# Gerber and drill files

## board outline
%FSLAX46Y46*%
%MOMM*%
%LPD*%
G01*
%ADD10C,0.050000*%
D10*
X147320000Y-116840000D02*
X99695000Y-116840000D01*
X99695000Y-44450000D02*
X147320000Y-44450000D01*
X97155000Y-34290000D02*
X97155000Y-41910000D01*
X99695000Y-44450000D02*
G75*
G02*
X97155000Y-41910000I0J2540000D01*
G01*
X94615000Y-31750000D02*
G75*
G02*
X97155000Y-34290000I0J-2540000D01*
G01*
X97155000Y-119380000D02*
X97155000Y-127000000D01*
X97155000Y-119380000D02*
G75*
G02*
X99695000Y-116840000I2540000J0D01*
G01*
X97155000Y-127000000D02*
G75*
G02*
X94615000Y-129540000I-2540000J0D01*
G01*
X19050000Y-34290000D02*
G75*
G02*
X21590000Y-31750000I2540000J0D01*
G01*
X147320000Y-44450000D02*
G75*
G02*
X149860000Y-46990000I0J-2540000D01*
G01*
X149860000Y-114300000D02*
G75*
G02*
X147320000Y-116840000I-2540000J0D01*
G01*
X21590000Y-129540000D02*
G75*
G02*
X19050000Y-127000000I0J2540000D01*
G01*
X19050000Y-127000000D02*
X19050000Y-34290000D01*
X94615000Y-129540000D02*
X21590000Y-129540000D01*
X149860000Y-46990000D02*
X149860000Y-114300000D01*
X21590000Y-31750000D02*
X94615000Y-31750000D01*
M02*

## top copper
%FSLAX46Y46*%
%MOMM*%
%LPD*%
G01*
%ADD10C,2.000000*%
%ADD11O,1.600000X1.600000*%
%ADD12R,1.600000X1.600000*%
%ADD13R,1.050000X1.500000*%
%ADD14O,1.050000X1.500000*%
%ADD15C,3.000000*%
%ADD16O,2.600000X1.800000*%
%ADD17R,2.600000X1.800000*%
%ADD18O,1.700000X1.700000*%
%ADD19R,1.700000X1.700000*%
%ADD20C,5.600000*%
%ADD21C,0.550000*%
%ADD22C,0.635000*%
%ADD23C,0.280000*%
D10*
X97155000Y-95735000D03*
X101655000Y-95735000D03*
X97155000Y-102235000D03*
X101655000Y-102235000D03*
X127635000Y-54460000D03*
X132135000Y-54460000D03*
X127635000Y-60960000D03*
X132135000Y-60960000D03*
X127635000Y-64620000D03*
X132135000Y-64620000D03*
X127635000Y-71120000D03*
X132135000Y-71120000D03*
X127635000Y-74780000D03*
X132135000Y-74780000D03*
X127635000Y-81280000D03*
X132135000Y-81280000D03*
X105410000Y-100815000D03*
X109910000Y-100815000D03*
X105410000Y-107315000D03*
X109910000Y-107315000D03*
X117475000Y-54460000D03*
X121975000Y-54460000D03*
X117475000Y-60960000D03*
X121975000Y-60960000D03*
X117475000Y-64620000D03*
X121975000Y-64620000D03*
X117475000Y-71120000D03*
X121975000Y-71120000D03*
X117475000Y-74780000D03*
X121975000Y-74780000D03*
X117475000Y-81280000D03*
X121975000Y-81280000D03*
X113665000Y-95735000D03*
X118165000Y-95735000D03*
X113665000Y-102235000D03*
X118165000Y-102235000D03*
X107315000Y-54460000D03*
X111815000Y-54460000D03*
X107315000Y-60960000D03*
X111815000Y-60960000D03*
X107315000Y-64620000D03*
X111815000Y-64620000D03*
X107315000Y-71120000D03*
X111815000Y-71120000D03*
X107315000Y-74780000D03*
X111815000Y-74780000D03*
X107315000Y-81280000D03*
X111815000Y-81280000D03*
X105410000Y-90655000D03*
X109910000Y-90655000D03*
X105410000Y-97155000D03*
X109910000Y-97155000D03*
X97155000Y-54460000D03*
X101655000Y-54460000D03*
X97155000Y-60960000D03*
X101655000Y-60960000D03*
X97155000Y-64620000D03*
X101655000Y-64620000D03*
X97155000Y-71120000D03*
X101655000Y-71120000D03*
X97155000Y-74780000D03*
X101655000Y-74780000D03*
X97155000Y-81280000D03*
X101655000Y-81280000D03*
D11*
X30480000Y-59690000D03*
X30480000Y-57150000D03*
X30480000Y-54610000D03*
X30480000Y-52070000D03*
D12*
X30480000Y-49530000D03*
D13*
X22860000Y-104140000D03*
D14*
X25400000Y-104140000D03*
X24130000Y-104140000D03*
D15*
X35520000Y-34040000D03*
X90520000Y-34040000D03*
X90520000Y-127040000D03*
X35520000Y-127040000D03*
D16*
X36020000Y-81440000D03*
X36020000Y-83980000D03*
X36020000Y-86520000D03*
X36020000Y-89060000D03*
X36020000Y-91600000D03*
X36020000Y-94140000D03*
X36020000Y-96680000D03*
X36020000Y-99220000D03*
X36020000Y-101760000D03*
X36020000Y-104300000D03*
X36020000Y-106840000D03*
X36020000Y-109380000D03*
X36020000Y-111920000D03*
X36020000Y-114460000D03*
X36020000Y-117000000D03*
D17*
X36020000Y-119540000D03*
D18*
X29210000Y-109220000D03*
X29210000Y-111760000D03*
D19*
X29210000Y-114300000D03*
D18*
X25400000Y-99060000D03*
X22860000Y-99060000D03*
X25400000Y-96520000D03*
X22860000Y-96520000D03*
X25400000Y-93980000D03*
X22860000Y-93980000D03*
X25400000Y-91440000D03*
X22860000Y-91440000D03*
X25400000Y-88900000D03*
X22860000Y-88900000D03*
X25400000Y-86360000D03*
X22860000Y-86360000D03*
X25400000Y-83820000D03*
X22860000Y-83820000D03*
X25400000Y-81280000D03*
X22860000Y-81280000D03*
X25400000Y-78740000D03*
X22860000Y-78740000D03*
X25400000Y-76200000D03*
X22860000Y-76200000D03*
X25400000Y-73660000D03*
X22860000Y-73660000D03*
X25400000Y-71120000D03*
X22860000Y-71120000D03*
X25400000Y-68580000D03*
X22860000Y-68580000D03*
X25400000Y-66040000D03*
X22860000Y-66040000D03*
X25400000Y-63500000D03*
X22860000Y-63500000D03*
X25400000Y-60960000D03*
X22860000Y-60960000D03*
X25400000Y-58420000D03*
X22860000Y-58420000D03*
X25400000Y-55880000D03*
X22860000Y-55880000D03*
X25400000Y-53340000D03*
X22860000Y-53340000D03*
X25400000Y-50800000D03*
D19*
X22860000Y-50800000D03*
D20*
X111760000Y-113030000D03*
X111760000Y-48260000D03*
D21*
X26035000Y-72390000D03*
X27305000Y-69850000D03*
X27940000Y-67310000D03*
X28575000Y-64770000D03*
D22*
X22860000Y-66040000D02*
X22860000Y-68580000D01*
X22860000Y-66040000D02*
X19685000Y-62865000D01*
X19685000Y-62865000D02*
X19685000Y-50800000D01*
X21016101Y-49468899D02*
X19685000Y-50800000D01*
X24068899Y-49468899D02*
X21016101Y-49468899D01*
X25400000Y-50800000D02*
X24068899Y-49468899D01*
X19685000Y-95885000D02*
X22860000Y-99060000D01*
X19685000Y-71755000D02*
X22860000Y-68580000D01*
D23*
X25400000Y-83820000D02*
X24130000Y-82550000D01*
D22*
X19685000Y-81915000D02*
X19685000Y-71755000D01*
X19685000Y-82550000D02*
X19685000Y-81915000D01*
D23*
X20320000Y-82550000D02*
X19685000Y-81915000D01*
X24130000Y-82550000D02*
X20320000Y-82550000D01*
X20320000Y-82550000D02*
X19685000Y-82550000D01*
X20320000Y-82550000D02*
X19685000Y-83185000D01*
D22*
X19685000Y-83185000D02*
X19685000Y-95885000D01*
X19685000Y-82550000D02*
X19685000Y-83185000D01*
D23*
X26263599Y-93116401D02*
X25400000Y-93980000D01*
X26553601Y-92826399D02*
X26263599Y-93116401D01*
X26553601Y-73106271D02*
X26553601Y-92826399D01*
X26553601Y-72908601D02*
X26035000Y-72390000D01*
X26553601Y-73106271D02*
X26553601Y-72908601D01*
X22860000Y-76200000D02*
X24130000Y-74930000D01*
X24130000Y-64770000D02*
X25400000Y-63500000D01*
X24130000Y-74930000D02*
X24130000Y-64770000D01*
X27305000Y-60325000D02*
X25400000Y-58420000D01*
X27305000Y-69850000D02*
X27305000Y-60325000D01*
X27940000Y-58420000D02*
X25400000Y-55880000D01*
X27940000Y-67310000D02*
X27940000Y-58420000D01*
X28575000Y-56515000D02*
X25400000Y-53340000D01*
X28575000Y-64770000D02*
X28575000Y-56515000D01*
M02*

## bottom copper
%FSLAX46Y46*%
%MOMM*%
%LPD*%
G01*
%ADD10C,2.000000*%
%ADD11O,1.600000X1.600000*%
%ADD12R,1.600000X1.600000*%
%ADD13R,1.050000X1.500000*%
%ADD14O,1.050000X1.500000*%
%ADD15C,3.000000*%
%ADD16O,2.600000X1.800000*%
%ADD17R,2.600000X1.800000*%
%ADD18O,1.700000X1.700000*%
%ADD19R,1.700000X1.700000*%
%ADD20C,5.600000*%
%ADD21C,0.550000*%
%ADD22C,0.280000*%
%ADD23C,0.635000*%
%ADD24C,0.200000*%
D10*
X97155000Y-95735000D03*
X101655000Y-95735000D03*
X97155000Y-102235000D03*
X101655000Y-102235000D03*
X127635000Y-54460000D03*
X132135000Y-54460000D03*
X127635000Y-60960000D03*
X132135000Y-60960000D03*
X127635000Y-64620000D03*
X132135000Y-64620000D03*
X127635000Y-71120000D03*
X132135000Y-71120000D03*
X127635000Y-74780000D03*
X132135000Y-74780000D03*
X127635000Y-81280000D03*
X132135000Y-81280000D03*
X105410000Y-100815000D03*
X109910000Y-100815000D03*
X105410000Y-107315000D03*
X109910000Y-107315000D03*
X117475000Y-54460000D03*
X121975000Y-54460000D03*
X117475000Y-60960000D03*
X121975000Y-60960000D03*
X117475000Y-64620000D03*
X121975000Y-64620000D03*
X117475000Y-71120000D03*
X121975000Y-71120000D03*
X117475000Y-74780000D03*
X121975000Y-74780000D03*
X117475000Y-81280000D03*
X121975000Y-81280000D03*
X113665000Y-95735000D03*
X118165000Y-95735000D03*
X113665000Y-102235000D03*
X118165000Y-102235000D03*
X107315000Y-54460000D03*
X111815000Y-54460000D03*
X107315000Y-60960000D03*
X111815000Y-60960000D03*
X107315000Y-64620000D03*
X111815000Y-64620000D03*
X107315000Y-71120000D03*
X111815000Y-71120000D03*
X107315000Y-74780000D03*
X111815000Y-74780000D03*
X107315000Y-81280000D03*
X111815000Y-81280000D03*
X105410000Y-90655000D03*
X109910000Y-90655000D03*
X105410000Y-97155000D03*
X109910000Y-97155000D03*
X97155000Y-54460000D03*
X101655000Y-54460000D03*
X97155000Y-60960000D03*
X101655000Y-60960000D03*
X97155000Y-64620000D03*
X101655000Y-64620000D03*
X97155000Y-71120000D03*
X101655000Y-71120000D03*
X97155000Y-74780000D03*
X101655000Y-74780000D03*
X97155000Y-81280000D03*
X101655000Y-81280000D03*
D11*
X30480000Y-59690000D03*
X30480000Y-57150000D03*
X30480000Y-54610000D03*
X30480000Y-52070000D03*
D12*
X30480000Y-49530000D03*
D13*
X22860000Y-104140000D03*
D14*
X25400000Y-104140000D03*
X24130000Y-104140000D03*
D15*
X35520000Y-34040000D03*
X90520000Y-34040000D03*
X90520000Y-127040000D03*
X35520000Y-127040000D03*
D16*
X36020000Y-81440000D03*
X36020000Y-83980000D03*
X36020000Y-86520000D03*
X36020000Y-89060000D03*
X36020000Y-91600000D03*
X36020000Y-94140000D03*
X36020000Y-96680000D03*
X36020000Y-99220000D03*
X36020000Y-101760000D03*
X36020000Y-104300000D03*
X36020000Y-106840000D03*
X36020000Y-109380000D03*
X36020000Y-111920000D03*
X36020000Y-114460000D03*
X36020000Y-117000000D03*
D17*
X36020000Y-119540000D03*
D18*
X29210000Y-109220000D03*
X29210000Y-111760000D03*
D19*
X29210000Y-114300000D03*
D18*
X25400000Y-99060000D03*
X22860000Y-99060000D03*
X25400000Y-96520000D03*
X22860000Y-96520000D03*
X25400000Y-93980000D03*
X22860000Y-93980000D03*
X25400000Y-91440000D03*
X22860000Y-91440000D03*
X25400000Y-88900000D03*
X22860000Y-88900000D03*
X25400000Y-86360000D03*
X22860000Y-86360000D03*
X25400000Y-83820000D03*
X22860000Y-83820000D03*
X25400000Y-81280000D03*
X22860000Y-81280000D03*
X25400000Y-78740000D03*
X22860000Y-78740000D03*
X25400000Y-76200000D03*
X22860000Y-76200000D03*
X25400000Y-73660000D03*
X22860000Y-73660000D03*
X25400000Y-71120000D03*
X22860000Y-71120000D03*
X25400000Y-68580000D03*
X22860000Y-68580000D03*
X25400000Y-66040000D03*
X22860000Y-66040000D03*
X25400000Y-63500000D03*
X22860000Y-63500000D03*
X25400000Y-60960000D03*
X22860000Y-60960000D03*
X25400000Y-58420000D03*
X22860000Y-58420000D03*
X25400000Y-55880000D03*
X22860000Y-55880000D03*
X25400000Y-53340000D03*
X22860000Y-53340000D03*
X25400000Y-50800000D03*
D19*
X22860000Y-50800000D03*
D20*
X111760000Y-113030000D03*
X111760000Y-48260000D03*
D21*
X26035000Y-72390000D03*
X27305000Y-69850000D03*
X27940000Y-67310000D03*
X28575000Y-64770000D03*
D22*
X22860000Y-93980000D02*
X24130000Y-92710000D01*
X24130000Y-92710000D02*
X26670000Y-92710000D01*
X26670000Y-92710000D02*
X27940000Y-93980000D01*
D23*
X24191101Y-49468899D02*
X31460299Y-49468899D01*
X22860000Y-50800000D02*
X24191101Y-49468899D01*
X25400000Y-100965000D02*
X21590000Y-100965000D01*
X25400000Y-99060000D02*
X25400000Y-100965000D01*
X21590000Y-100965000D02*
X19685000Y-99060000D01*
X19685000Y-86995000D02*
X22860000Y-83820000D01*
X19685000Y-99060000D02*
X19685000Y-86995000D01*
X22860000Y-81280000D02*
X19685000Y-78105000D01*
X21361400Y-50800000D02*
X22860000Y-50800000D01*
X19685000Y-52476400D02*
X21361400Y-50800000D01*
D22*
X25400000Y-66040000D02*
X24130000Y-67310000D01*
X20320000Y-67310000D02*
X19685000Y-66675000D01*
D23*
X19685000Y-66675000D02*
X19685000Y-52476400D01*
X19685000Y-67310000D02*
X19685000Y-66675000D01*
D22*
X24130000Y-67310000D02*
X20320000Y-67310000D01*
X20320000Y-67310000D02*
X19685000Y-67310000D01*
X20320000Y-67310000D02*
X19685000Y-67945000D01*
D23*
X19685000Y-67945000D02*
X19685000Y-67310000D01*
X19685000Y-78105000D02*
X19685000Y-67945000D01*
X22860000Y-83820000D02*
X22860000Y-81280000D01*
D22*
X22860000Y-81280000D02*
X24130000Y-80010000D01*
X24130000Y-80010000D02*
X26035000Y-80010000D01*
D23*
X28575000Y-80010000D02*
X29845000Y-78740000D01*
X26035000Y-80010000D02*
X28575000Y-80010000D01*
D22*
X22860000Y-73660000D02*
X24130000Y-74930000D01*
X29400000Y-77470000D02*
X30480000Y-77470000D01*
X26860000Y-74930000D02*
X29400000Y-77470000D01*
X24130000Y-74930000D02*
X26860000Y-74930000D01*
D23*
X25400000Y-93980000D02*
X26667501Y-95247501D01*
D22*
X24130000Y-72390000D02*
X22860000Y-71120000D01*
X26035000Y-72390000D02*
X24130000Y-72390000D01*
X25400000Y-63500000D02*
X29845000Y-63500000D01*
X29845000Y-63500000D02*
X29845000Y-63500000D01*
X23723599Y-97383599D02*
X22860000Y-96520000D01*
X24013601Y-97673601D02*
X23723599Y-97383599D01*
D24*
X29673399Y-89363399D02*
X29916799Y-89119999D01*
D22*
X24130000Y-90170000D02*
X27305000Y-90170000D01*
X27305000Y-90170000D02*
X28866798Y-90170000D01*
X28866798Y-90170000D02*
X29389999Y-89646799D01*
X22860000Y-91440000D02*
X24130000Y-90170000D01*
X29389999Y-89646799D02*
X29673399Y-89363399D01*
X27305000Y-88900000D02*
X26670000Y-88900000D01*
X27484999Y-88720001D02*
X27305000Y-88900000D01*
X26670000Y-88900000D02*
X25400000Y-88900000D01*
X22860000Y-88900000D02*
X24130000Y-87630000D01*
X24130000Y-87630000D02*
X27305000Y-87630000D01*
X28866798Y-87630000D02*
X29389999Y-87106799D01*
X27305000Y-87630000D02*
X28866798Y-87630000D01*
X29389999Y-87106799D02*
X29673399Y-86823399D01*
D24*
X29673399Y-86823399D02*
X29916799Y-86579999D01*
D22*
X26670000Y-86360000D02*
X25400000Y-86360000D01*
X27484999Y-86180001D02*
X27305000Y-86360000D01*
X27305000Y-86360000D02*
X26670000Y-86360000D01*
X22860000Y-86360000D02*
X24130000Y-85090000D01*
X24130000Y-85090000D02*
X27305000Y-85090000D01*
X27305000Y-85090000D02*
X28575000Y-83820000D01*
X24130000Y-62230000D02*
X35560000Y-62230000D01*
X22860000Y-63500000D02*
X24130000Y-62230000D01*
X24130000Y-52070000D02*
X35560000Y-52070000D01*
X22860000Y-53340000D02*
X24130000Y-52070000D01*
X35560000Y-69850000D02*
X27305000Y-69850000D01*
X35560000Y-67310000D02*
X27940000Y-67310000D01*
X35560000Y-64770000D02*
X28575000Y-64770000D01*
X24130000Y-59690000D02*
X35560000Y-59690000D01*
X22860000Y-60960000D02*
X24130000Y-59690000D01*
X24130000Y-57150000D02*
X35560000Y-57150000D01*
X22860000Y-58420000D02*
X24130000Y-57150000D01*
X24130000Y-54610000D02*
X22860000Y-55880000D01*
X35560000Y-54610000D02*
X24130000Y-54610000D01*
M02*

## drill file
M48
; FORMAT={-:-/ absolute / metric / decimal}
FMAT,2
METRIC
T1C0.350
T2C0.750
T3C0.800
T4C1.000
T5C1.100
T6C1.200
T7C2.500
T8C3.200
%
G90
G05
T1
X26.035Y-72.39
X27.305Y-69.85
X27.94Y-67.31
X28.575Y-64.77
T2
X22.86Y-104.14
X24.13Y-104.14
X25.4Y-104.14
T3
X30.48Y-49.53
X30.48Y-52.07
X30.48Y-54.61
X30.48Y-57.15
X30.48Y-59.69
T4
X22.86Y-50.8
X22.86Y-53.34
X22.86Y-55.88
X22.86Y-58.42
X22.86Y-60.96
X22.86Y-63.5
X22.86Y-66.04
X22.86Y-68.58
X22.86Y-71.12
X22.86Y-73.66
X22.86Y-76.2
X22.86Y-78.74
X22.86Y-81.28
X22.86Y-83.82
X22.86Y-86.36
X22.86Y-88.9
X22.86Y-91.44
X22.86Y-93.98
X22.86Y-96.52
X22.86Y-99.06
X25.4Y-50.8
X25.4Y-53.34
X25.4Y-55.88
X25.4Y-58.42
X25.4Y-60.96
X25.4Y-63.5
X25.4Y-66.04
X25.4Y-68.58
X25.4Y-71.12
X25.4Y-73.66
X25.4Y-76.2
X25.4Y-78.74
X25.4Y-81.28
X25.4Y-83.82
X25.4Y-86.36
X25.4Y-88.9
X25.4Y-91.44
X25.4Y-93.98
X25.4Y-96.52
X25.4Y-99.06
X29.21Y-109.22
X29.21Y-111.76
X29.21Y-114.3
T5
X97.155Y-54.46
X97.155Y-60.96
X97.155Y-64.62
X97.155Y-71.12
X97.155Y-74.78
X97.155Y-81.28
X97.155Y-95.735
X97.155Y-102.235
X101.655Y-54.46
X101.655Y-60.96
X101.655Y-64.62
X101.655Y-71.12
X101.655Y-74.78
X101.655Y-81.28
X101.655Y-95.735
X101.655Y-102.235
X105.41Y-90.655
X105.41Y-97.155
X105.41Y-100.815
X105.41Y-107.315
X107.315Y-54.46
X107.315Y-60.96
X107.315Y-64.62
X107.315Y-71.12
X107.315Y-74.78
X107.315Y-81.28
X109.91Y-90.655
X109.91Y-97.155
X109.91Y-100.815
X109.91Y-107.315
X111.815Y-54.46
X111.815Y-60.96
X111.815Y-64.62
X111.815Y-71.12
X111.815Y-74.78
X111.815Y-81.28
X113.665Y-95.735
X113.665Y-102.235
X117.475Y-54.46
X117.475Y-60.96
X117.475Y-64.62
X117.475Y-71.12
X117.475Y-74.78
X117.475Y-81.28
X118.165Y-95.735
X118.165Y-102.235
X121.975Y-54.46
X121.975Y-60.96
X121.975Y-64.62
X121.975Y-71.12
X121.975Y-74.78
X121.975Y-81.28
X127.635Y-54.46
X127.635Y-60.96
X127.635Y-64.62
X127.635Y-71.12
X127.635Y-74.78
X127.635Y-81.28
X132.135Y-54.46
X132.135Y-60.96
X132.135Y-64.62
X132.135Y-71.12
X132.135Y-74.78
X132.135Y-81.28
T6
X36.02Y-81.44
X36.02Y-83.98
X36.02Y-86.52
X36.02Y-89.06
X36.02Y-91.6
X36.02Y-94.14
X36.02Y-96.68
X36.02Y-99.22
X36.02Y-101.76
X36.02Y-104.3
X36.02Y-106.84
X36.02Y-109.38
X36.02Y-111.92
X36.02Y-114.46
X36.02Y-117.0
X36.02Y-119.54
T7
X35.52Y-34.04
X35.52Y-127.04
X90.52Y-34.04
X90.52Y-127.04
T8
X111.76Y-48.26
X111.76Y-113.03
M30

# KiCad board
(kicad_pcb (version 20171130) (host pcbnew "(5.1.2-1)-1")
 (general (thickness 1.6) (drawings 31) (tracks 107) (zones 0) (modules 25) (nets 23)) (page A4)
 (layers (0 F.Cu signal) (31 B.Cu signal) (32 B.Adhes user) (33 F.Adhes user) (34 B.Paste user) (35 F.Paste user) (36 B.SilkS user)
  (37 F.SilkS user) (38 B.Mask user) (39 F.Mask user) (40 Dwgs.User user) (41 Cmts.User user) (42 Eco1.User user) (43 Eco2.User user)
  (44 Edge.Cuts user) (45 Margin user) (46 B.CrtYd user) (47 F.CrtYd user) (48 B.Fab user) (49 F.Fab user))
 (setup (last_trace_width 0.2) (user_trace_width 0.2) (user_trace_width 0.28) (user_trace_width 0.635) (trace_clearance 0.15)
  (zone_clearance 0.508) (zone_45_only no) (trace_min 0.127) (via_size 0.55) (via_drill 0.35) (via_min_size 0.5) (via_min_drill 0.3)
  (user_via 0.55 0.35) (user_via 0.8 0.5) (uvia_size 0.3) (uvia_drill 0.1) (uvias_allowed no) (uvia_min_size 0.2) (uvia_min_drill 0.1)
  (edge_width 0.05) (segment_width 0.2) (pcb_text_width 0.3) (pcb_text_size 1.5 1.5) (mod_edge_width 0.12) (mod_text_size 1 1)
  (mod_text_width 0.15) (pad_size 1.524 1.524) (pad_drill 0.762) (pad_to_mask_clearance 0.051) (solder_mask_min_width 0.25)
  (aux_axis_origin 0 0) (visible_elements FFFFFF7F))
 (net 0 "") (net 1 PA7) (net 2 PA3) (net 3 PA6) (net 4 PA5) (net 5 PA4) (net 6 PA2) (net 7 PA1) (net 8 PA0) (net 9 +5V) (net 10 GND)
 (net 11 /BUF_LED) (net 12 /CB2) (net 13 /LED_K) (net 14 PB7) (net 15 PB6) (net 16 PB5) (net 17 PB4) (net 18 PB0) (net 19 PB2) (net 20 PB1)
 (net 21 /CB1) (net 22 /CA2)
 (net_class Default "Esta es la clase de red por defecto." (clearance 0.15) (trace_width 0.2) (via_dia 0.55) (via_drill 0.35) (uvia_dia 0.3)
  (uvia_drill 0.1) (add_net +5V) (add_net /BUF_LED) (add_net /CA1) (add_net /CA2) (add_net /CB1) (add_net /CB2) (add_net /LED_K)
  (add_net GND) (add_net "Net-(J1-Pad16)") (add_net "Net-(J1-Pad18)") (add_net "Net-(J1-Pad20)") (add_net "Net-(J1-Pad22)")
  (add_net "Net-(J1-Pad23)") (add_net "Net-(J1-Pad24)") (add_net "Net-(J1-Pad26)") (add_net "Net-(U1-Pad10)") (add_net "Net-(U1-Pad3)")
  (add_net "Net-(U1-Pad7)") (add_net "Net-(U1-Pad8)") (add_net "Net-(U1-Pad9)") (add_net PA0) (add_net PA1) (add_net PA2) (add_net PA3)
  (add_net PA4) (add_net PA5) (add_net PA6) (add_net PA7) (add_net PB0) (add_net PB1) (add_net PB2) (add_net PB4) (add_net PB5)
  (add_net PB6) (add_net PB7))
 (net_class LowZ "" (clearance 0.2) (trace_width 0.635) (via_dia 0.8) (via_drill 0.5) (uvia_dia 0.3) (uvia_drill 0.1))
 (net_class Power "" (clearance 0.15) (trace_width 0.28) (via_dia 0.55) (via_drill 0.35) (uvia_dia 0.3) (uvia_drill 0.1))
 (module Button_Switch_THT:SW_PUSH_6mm (layer F.Cu) (at 97.155 102.235 90)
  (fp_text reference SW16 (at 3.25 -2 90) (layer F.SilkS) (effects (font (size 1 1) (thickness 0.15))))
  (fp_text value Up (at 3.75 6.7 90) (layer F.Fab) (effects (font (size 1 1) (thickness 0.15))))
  (pad 1 thru_hole circle (at 6.5 0 180) (size 2 2) (drill 1.1) (layers *.Cu *.Mask) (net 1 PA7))
  (pad 2 thru_hole circle (at 6.5 4.5 180) (size 2 2) (drill 1.1) (layers *.Cu *.Mask) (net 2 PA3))
  (pad 1 thru_hole circle (at 0 0 180) (size 2 2) (drill 1.1) (layers *.Cu *.Mask) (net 1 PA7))
  (pad 2 thru_hole circle (at 0 4.5 180) (size 2 2) (drill 1.1) (layers *.Cu *.Mask) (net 2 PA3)))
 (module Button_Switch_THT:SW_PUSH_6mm (layer F.Cu) (at 127.635 60.96 90)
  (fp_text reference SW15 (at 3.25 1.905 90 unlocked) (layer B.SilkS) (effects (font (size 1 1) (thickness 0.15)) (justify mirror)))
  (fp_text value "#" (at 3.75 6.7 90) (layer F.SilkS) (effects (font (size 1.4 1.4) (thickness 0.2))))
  (pad 1 thru_hole circle (at 6.5 0 180) (size 2 2) (drill 1.1) (layers *.Cu *.Mask) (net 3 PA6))
  (pad 2 thru_hole circle (at 6.5 4.5 180) (size 2 2) (drill 1.1) (layers *.Cu *.Mask) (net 2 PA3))
  (pad 1 thru_hole circle (at 0 0 180) (size 2 2) (drill 1.1) (layers *.Cu *.Mask) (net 3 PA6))
  (pad 2 thru_hole circle (at 0 4.5 180) (size 2 2) (drill 1.1) (layers *.Cu *.Mask) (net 2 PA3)))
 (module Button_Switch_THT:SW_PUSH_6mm (layer F.Cu) (at 127.635 71.12 90)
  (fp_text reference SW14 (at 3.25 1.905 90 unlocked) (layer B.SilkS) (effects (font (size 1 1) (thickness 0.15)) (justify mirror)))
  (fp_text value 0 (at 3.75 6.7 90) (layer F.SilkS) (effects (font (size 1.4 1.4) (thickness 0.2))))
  (pad 1 thru_hole circle (at 6.5 0 180) (size 2 2) (drill 1.1) (layers *.Cu *.Mask) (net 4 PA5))
  (pad 2 thru_hole circle (at 6.5 4.5 180) (size 2 2) (drill 1.1) (layers *.Cu *.Mask) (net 2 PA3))
  (pad 1 thru_hole circle (at 0 0 180) (size 2 2) (drill 1.1) (layers *.Cu *.Mask) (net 4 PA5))
  (pad 2 thru_hole circle (at 0 4.5 180) (size 2 2) (drill 1.1) (layers *.Cu *.Mask) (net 2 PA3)))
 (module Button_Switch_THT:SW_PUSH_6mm (layer F.Cu) (at 127.635 81.28 90)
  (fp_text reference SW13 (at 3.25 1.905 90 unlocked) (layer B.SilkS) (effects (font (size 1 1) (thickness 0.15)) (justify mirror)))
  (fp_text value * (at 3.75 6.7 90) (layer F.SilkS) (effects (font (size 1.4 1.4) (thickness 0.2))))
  (pad 1 thru_hole circle (at 6.5 0 180) (size 2 2) (drill 1.1) (layers *.Cu *.Mask) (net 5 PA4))
  (pad 2 thru_hole circle (at 6.5 4.5 180) (size 2 2) (drill 1.1) (layers *.Cu *.Mask) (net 2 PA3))
  (pad 1 thru_hole circle (at 0 0 180) (size 2 2) (drill 1.1) (layers *.Cu *.Mask) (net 5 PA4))
  (pad 2 thru_hole circle (at 0 4.5 180) (size 2 2) (drill 1.1) (layers *.Cu *.Mask) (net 2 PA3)))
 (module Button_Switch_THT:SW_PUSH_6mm (layer F.Cu) (at 105.41 107.315 90)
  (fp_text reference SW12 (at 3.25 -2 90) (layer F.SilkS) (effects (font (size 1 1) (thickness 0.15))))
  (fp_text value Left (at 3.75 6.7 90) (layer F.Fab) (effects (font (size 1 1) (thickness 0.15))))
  (pad 1 thru_hole circle (at 6.5 0 180) (size 2 2) (drill 1.1) (layers *.Cu *.Mask) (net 1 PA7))
  (pad 2 thru_hole circle (at 6.5 4.5 180) (size 2 2) (drill 1.1) (layers *.Cu *.Mask) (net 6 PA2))
  (pad 1 thru_hole circle (at 0 0 180) (size 2 2) (drill 1.1) (layers *.Cu *.Mask) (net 1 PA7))
  (pad 2 thru_hole circle (at 0 4.5 180) (size 2 2) (drill 1.1) (layers *.Cu *.Mask) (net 6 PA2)))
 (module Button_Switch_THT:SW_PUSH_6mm (layer F.Cu) (at 117.475 60.96 90)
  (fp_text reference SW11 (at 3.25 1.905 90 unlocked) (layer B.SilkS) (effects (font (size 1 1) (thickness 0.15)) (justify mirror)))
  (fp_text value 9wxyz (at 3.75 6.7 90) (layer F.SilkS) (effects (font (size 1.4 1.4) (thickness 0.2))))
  (pad 1 thru_hole circle (at 6.5 0 180) (size 2 2) (drill 1.1) (layers *.Cu *.Mask) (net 3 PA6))
  (pad 2 thru_hole circle (at 6.5 4.5 180) (size 2 2) (drill 1.1) (layers *.Cu *.Mask) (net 6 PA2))
  (pad 1 thru_hole circle (at 0 0 180) (size 2 2) (drill 1.1) (layers *.Cu *.Mask) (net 3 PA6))
  (pad 2 thru_hole circle (at 0 4.5 180) (size 2 2) (drill 1.1) (layers *.Cu *.Mask) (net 6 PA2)))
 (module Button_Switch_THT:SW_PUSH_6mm (layer F.Cu) (at 117.475 71.12 90)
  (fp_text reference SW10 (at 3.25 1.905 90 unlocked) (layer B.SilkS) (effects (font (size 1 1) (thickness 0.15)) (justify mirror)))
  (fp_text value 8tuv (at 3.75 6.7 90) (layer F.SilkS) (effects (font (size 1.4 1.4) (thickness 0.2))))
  (pad 1 thru_hole circle (at 6.5 0 180) (size 2 2) (drill 1.1) (layers *.Cu *.Mask) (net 4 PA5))
  (pad 2 thru_hole circle (at 6.5 4.5 180) (size 2 2) (drill 1.1) (layers *.Cu *.Mask) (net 6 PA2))
  (pad 1 thru_hole circle (at 0 0 180) (size 2 2) (drill 1.1) (layers *.Cu *.Mask) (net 4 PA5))
  (pad 2 thru_hole circle (at 0 4.5 180) (size 2 2) (drill 1.1) (layers *.Cu *.Mask) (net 6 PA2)))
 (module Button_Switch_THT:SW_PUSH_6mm (layer F.Cu) (at 117.475 81.28 90)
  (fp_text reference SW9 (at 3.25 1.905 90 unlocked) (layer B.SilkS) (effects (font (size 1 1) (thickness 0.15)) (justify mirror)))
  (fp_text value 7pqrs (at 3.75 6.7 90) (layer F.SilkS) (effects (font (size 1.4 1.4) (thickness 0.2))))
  (pad 1 thru_hole circle (at 6.5 0 180) (size 2 2) (drill 1.1) (layers *.Cu *.Mask) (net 5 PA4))
  (pad 2 thru_hole circle (at 6.5 4.5 180) (size 2 2) (drill 1.1) (layers *.Cu *.Mask) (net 6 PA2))
  (pad 1 thru_hole circle (at 0 0 180) (size 2 2) (drill 1.1) (layers *.Cu *.Mask) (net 5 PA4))
  (pad 2 thru_hole circle (at 0 4.5 180) (size 2 2) (drill 1.1) (layers *.Cu *.Mask) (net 6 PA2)))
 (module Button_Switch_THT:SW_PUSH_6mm (layer F.Cu) (at 113.665 102.235 90)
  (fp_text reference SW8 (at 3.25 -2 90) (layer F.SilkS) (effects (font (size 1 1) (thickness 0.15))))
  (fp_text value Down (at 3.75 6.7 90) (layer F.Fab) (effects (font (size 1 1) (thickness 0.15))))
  (pad 1 thru_hole circle (at 6.5 0 180) (size 2 2) (drill 1.1) (layers *.Cu *.Mask) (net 1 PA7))
  (pad 2 thru_hole circle (at 6.5 4.5 180) (size 2 2) (drill 1.1) (layers *.Cu *.Mask) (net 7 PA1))
  (pad 1 thru_hole circle (at 0 0 180) (size 2 2) (drill 1.1) (layers *.Cu *.Mask) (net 1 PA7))
  (pad 2 thru_hole circle (at 0 4.5 180) (size 2 2) (drill 1.1) (layers *.Cu *.Mask) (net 7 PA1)))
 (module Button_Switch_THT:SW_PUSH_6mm (layer F.Cu) (at 107.315 60.96 90)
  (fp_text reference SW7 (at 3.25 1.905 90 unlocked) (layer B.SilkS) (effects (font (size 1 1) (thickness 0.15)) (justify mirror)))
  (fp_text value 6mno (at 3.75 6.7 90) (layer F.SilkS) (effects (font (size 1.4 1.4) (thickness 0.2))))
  (pad 1 thru_hole circle (at 6.5 0 180) (size 2 2) (drill 1.1) (layers *.Cu *.Mask) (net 3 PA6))
  (pad 2 thru_hole circle (at 6.5 4.5 180) (size 2 2) (drill 1.1) (layers *.Cu *.Mask) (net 7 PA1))
  (pad 1 thru_hole circle (at 0 0 180) (size 2 2) (drill 1.1) (layers *.Cu *.Mask) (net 3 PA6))
  (pad 2 thru_hole circle (at 0 4.5 180) (size 2 2) (drill 1.1) (layers *.Cu *.Mask) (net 7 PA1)))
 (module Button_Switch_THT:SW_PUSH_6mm (layer F.Cu) (at 107.315 71.12 90)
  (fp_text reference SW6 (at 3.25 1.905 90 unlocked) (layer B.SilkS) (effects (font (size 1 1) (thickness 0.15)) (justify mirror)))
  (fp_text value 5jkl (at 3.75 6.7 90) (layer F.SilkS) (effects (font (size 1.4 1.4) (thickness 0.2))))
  (pad 1 thru_hole circle (at 6.5 0 180) (size 2 2) (drill 1.1) (layers *.Cu *.Mask) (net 4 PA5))
  (pad 2 thru_hole circle (at 6.5 4.5 180) (size 2 2) (drill 1.1) (layers *.Cu *.Mask) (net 7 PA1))
  (pad 1 thru_hole circle (at 0 0 180) (size 2 2) (drill 1.1) (layers *.Cu *.Mask) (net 4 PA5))
  (pad 2 thru_hole circle (at 0 4.5 180) (size 2 2) (drill 1.1) (layers *.Cu *.Mask) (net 7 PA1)))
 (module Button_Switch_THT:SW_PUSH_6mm (layer F.Cu) (at 107.315 81.28 90)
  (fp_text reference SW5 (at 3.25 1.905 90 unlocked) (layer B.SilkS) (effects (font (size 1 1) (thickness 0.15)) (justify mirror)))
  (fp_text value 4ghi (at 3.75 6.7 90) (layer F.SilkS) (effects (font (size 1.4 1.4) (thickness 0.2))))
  (pad 1 thru_hole circle (at 6.5 0 180) (size 2 2) (drill 1.1) (layers *.Cu *.Mask) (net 5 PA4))
  (pad 2 thru_hole circle (at 6.5 4.5 180) (size 2 2) (drill 1.1) (layers *.Cu *.Mask) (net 7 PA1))
  (pad 1 thru_hole circle (at 0 0 180) (size 2 2) (drill 1.1) (layers *.Cu *.Mask) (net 5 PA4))
  (pad 2 thru_hole circle (at 0 4.5 180) (size 2 2) (drill 1.1) (layers *.Cu *.Mask) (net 7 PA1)))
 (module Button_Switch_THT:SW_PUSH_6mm (layer F.Cu) (at 105.41 97.155 90)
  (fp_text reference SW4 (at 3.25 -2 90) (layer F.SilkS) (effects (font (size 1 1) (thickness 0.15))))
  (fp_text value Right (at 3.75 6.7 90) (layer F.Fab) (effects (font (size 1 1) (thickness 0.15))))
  (pad 1 thru_hole circle (at 6.5 0 180) (size 2 2) (drill 1.1) (layers *.Cu *.Mask) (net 1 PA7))
  (pad 2 thru_hole circle (at 6.5 4.5 180) (size 2 2) (drill 1.1) (layers *.Cu *.Mask) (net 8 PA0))
  (pad 1 thru_hole circle (at 0 0 180) (size 2 2) (drill 1.1) (layers *.Cu *.Mask) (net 1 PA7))
  (pad 2 thru_hole circle (at 0 4.5 180) (size 2 2) (drill 1.1) (layers *.Cu *.Mask) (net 8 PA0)))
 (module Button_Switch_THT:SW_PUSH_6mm (layer F.Cu) (at 97.155 60.96 90)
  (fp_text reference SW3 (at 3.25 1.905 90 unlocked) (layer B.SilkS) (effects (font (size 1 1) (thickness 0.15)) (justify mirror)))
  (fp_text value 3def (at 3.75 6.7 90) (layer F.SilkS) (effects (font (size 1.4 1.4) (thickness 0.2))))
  (pad 1 thru_hole circle (at 6.5 0 180) (size 2 2) (drill 1.1) (layers *.Cu *.Mask) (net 3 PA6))
  (pad 2 thru_hole circle (at 6.5 4.5 180) (size 2 2) (drill 1.1) (layers *.Cu *.Mask) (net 8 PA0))
  (pad 1 thru_hole circle (at 0 0 180) (size 2 2) (drill 1.1) (layers *.Cu *.Mask) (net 3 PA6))
  (pad 2 thru_hole circle (at 0 4.5 180) (size 2 2) (drill 1.1) (layers *.Cu *.Mask) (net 8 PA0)))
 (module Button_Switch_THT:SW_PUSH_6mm (layer F.Cu) (at 97.155 71.12 90)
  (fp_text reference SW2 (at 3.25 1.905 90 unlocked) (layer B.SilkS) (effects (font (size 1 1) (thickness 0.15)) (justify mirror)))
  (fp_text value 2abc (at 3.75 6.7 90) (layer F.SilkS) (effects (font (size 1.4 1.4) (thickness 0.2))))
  (pad 1 thru_hole circle (at 6.5 0 180) (size 2 2) (drill 1.1) (layers *.Cu *.Mask) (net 4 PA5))
  (pad 2 thru_hole circle (at 6.5 4.5 180) (size 2 2) (drill 1.1) (layers *.Cu *.Mask) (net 8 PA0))
  (pad 1 thru_hole circle (at 0 0 180) (size 2 2) (drill 1.1) (layers *.Cu *.Mask) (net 4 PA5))
  (pad 2 thru_hole circle (at 0 4.5 180) (size 2 2) (drill 1.1) (layers *.Cu *.Mask) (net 8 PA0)))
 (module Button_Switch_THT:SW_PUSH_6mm (layer F.Cu) (at 97.155 81.28 90)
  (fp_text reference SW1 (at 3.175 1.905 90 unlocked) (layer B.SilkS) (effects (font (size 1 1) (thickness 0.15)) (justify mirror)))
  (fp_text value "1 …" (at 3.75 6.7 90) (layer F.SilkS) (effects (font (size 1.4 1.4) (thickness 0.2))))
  (pad 1 thru_hole circle (at 6.5 0 180) (size 2 2) (drill 1.1) (layers *.Cu *.Mask) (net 5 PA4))
  (pad 2 thru_hole circle (at 6.5 4.5 180) (size 2 2) (drill 1.1) (layers *.Cu *.Mask) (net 8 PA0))
  (pad 1 thru_hole circle (at 0 0 180) (size 2 2) (drill 1.1) (layers *.Cu *.Mask) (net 5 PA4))
  (pad 2 thru_hole circle (at 0 4.5 180) (size 2 2) (drill 1.1) (layers *.Cu *.Mask) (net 8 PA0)))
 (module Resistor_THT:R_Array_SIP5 (layer F.Cu) (at 30.48 49.53 270)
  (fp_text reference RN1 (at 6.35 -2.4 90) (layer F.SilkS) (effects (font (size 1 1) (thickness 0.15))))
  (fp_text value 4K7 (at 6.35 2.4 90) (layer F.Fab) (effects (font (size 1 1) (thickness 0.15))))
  (pad 5 thru_hole oval (at 10.16 0 270) (size 1.6 1.6) (drill 0.8) (layers *.Cu *.Mask) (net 2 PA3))
  (pad 4 thru_hole oval (at 7.62 0 270) (size 1.6 1.6) (drill 0.8) (layers *.Cu *.Mask) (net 6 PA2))
  (pad 3 thru_hole oval (at 5.08 0 270) (size 1.6 1.6) (drill 0.8) (layers *.Cu *.Mask) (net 7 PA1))
  (pad 2 thru_hole oval (at 2.54 0 270) (size 1.6 1.6) (drill 0.8) (layers *.Cu *.Mask) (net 8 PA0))
  (pad 1 thru_hole rect (at 0 0 270) (size 1.6 1.6) (drill 0.8) (layers *.Cu *.Mask) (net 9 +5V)))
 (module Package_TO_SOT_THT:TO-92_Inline (layer F.Cu) (at 22.86 104.14)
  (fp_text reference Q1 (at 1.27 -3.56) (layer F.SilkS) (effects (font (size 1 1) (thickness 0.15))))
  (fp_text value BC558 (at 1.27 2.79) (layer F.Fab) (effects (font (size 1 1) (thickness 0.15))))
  (pad 1 thru_hole rect (at 0 0) (size 1.05 1.5) (drill 0.75) (layers *.Cu *.Mask) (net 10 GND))
  (pad 3 thru_hole oval (at 2.54 0) (size 1.05 1.5) (drill 0.75) (layers *.Cu *.Mask) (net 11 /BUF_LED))
  (pad 2 thru_hole oval (at 1.27 0) (size 1.05 1.5) (drill 0.75) (layers *.Cu *.Mask) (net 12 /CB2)))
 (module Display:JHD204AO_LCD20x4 (layer F.Cu) (at 33.02 129.54 90)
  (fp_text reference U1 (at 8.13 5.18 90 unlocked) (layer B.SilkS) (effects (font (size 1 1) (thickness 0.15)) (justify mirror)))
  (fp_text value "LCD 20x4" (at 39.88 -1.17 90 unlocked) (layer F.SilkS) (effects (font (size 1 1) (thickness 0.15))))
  (pad "" thru_hole circle (at 95.5 2.5 90) (size 3 3) (drill 2.5) (layers *.Cu *.Mask))
  (pad "" thru_hole circle (at 95.5 57.5 90) (size 3 3) (drill 2.5) (layers *.Cu *.Mask))
  (pad "" thru_hole circle (at 2.5 57.5 90) (size 3 3) (drill 2.5) (layers *.Cu *.Mask))
  (pad "" thru_hole circle (at 2.5 2.5 90) (size 3 3) (drill 2.5) (layers *.Cu *.Mask))
  (pad 16 thru_hole oval (at 48.1 3 90) (size 1.8 2.6) (drill 1.2) (layers *.Cu *.Mask) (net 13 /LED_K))
  (pad 15 thru_hole oval (at 45.56 3 90) (size 1.8 2.6) (drill 1.2) (layers *.Cu *.Mask) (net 9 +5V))
  (pad 14 thru_hole oval (at 43.02 3 90) (size 1.8 2.6) (drill 1.2) (layers *.Cu *.Mask) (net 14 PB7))
  (pad 13 thru_hole oval (at 40.48 3 90) (size 1.8 2.6) (drill 1.2) (layers *.Cu *.Mask) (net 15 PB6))
  (pad 12 thru_hole oval (at 37.94 3 90) (size 1.8 2.6) (drill 1.2) (layers *.Cu *.Mask) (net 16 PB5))
  (pad 11 thru_hole oval (at 35.4 3 90) (size 1.8 2.6) (drill 1.2) (layers *.Cu *.Mask) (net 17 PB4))
  (pad 10 thru_hole oval (at 32.86 3 90) (size 1.8 2.6) (drill 1.2) (layers *.Cu *.Mask))
  (pad 9 thru_hole oval (at 30.32 3 90) (size 1.8 2.6) (drill 1.2) (layers *.Cu *.Mask))
  (pad 8 thru_hole oval (at 27.78 3 90) (size 1.8 2.6) (drill 1.2) (layers *.Cu *.Mask))
  (pad 7 thru_hole oval (at 25.24 3 90) (size 1.8 2.6) (drill 1.2) (layers *.Cu *.Mask))
  (pad 6 thru_hole oval (at 22.7 3 90) (size 1.8 2.6) (drill 1.2) (layers *.Cu *.Mask) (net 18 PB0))
  (pad 5 thru_hole oval (at 20.16 3 90) (size 1.8 2.6) (drill 1.2) (layers *.Cu *.Mask) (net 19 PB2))
  (pad 4 thru_hole oval (at 17.62 3 90) (size 1.8 2.6) (drill 1.2) (layers *.Cu *.Mask) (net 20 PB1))
  (pad 3 thru_hole oval (at 15.08 3 90) (size 1.8 2.6) (drill 1.2) (layers *.Cu *.Mask))
  (pad 2 thru_hole oval (at 12.54 3 90) (size 1.8 2.6) (drill 1.2) (layers *.Cu *.Mask) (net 9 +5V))
  (pad 1 thru_hole rect (at 10 3 90) (size 1.8 2.6) (drill 1.2) (layers *.Cu *.Mask) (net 10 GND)))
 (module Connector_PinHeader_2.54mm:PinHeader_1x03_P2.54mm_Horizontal (layer F.Cu) (at 29.21 114.3 180)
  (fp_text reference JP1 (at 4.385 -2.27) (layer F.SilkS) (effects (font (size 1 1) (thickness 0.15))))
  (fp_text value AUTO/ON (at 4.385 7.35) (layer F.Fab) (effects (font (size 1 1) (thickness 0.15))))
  (pad 3 thru_hole oval (at 0 5.08 180) (size 1.7 1.7) (drill 1) (layers *.Cu *.Mask) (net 10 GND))
  (pad 2 thru_hole oval (at 0 2.54 180) (size 1.7 1.7) (drill 1) (layers *.Cu *.Mask) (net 13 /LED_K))
  (pad 1 thru_hole rect (at 0 0 180) (size 1.7 1.7) (drill 1) (layers *.Cu *.Mask) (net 11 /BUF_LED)))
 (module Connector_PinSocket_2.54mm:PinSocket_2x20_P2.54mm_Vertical (layer B.Cu) (at 22.86 50.8 180)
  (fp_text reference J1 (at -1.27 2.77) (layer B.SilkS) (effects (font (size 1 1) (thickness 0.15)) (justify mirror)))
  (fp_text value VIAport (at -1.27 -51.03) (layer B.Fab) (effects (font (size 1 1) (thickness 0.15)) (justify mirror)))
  (pad 40 thru_hole oval (at -2.54 -48.26 180) (size 1.7 1.7) (drill 1) (layers *.Cu *.Mask) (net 9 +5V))
  (pad 39 thru_hole oval (at 0 -48.26 180) (size 1.7 1.7) (drill 1) (layers *.Cu *.Mask) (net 10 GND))
  (pad 38 thru_hole oval (at -2.54 -45.72 180) (size 1.7 1.7) (drill 1) (layers *.Cu *.Mask) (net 12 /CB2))
  (pad 37 thru_hole oval (at 0 -45.72 180) (size 1.7 1.7) (drill 1) (layers *.Cu *.Mask) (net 17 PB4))
  (pad 36 thru_hole oval (at -2.54 -43.18 180) (size 1.7 1.7) (drill 1) (layers *.Cu *.Mask) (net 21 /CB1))
  (pad 35 thru_hole oval (at 0 -43.18 180) (size 1.7 1.7) (drill 1) (layers *.Cu *.Mask))
  (pad 34 thru_hole oval (at -2.54 -40.64 180) (size 1.7 1.7) (drill 1) (layers *.Cu *.Mask) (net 14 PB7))
  (pad 33 thru_hole oval (at 0 -40.64 180) (size 1.7 1.7) (drill 1) (layers *.Cu *.Mask) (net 19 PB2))
  (pad 32 thru_hole oval (at -2.54 -38.1 180) (size 1.7 1.7) (drill 1) (layers *.Cu *.Mask) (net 15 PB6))
  (pad 31 thru_hole oval (at 0 -38.1 180) (size 1.7 1.7) (drill 1) (layers *.Cu *.Mask) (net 20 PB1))
  (pad 30 thru_hole oval (at -2.54 -35.56 180) (size 1.7 1.7) (drill 1) (layers *.Cu *.Mask) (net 16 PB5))
  (pad 29 thru_hole oval (at 0 -35.56 180) (size 1.7 1.7) (drill 1) (layers *.Cu *.Mask) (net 18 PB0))
  (pad 28 thru_hole oval (at -2.54 -33.02 180) (size 1.7 1.7) (drill 1) (layers *.Cu *.Mask) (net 10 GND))
  (pad 27 thru_hole oval (at 0 -33.02 180) (size 1.7 1.7) (drill 1) (layers *.Cu *.Mask) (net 9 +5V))
  (pad 26 thru_hole oval (at -2.54 -30.48 180) (size 1.7 1.7) (drill 1) (layers *.Cu *.Mask))
  (pad 25 thru_hole oval (at 0 -30.48 180) (size 1.7 1.7) (drill 1) (layers *.Cu *.Mask) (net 9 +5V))
  (pad 24 thru_hole oval (at -2.54 -27.94 180) (size 1.7 1.7) (drill 1) (layers *.Cu *.Mask))
  (pad 23 thru_hole oval (at 0 -27.94 180) (size 1.7 1.7) (drill 1) (layers *.Cu *.Mask))
  (pad 22 thru_hole oval (at -2.54 -25.4 180) (size 1.7 1.7) (drill 1) (layers *.Cu *.Mask))
  (pad 21 thru_hole oval (at 0 -25.4 180) (size 1.7 1.7) (drill 1) (layers *.Cu *.Mask) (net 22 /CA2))
  (pad 20 thru_hole oval (at -2.54 -22.86 180) (size 1.7 1.7) (drill 1) (layers *.Cu *.Mask))
  (pad 19 thru_hole oval (at 0 -22.86 180) (size 1.7 1.7) (drill 1) (layers *.Cu *.Mask) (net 12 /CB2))
  (pad 18 thru_hole oval (at -2.54 -20.32 180) (size 1.7 1.7) (drill 1) (layers *.Cu *.Mask))
  (pad 17 thru_hole oval (at 0 -20.32 180) (size 1.7 1.7) (drill 1) (layers *.Cu *.Mask) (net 21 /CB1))
  (pad 16 thru_hole oval (at -2.54 -17.78 180) (size 1.7 1.7) (drill 1) (layers *.Cu *.Mask))
  (pad 15 thru_hole oval (at 0 -17.78 180) (size 1.7 1.7) (drill 1) (layers *.Cu *.Mask) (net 10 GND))
  (pad 14 thru_hole oval (at -2.54 -15.24 180) (size 1.7 1.7) (drill 1) (layers *.Cu *.Mask) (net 9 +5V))
  (pad 13 thru_hole oval (at 0 -15.24 180) (size 1.7 1.7) (drill 1) (layers *.Cu *.Mask) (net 10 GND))
  (pad 12 thru_hole oval (at -2.54 -12.7 180) (size 1.7 1.7) (drill 1) (layers *.Cu *.Mask) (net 22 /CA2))
  (pad 11 thru_hole oval (at 0 -12.7 180) (size 1.7 1.7) (drill 1) (layers *.Cu *.Mask) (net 5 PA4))
  (pad 10 thru_hole oval (at -2.54 -10.16 180) (size 1.7 1.7) (drill 1) (layers *.Cu *.Mask))
  (pad 9 thru_hole oval (at 0 -10.16 180) (size 1.7 1.7) (drill 1) (layers *.Cu *.Mask) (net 2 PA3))
  (pad 8 thru_hole oval (at -2.54 -7.62 180) (size 1.7 1.7) (drill 1) (layers *.Cu *.Mask) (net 1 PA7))
  (pad 7 thru_hole oval (at 0 -7.62 180) (size 1.7 1.7) (drill 1) (layers *.Cu *.Mask) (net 6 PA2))
  (pad 6 thru_hole oval (at -2.54 -5.08 180) (size 1.7 1.7) (drill 1) (layers *.Cu *.Mask) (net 3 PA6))
  (pad 5 thru_hole oval (at 0 -5.08 180) (size 1.7 1.7) (drill 1) (layers *.Cu *.Mask) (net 7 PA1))
  (pad 4 thru_hole oval (at -2.54 -2.54 180) (size 1.7 1.7) (drill 1) (layers *.Cu *.Mask) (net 4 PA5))
  (pad 3 thru_hole oval (at 0 -2.54 180) (size 1.7 1.7) (drill 1) (layers *.Cu *.Mask) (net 8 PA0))
  (pad 2 thru_hole oval (at -2.54 0 180) (size 1.7 1.7) (drill 1) (layers *.Cu *.Mask) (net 10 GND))
  (pad 1 thru_hole rect (at 0 0 180) (size 1.7 1.7) (drill 1) (layers *.Cu *.Mask) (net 9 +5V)))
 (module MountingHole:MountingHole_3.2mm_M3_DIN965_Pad (layer F.Cu) (at 111.76 113.03)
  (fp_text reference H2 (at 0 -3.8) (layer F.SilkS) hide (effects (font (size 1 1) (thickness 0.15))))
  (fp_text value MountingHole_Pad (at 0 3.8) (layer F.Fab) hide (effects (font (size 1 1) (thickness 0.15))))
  (pad 1 thru_hole circle (at 0 0) (size 5.6 5.6) (drill 3.2) (layers *.Cu *.Mask) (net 10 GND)))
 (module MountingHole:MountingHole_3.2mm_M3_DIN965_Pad (layer F.Cu) (at 111.76 48.26)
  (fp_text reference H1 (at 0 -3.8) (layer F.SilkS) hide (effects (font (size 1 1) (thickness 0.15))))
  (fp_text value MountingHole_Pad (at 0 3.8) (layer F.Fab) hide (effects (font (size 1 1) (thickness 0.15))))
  (pad 1 thru_hole circle (at 0 0) (size 5.6 5.6) (drill 3.2) (layers *.Cu *.Mask) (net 10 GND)))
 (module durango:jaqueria (layer F.Cu) (at 143.51 55.88 90)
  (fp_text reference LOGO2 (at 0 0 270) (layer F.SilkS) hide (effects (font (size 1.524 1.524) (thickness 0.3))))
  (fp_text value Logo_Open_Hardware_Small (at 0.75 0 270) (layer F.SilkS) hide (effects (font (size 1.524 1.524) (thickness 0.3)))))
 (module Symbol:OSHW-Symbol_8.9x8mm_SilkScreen (layer B.Cu) (at 53.34 88.9 180)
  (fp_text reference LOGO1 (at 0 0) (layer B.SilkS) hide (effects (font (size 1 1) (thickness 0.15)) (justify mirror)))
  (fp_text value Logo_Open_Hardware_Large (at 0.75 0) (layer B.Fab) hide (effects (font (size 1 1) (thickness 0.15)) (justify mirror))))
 (gr_line (start 147.32 116.84) (end 99.695 116.84) (layer Edge.Cuts) (width 0.05))
 (gr_line (start 99.695 44.45) (end 147.32 44.45) (layer Edge.Cuts) (width 0.05))
 (gr_line (start 97.155 34.29) (end 97.155 41.91) (layer Edge.Cuts) (width 0.05))
 (gr_arc (start 99.695 41.91) (end 97.155 41.91) (angle -90) (layer Edge.Cuts) (width 0.05))
 (gr_arc (start 94.615 34.29) (end 97.155 34.29) (angle -90) (layer Edge.Cuts) (width 0.05))
 (gr_line (start 97.155 119.38) (end 97.155 127) (layer Edge.Cuts) (width 0.05))
 (gr_arc (start 99.695 119.38) (end 99.695 116.84) (angle -90) (layer Edge.Cuts) (width 0.05))
 (gr_arc (start 94.615 127) (end 94.615 129.54) (angle -90) (layer Edge.Cuts) (width 0.05))
 (gr_arc (start 21.59 34.29) (end 21.59 31.75) (angle -90) (layer Edge.Cuts) (width 0.05))
 (gr_arc (start 147.32 46.99) (end 149.86 46.99) (angle -90) (layer Edge.Cuts) (width 0.05))
 (gr_arc (start 147.32 114.3) (end 147.32 116.84) (angle -90) (layer Edge.Cuts) (width 0.05))
 (gr_arc (start 21.59 127) (end 19.05 127) (angle -90) (layer Edge.Cuts) (width 0.05))
 (gr_line (start 19.05 127) (end 19.05 34.29) (layer Edge.Cuts) (width 0.05))
 (gr_line (start 94.615 129.54) (end 21.59 129.54) (layer Edge.Cuts) (width 0.05))
 (gr_line (start 149.86 46.99) (end 149.86 114.3) (layer Edge.Cuts) (width 0.05))
 (gr_line (start 21.59 31.75) (end 94.615 31.75) (layer Edge.Cuts) (width 0.05))
 (segment (start 22.86 93.98) (end 24.13 92.71) (width 0.28) (layer B.Cu) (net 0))
 (segment (start 24.13 92.71) (end 26.67 92.71) (width 0.28) (layer B.Cu) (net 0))
 (segment (start 26.67 92.71) (end 27.94 93.98) (width 0.28) (layer B.Cu) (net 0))
 (segment (start 22.86 66.04) (end 22.86 68.58) (width 0.635) (layer F.Cu) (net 10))
 (segment (start 22.86 66.04) (end 19.685 62.865) (width 0.635) (layer F.Cu) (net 10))
 (segment (start 19.685 62.865) (end 19.685 50.8) (width 0.635) (layer F.Cu) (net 10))
 (segment (start 21.016101 49.468899) (end 19.685 50.8) (width 0.635) (layer F.Cu) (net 10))
 (segment (start 24.068899 49.468899) (end 21.016101 49.468899) (width 0.635) (layer F.Cu) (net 10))
 (segment (start 25.4 50.8) (end 24.068899 49.468899) (width 0.635) (layer F.Cu) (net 10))
 (segment (start 19.685 95.885) (end 22.86 99.06) (width 0.635) (layer F.Cu) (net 10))
 (segment (start 19.685 71.755) (end 22.86 68.58) (width 0.635) (layer F.Cu) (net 10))
 (segment (start 25.4 83.82) (end 24.13 82.55) (width 0.28) (layer F.Cu) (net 10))
 (segment (start 19.685 81.915) (end 19.685 71.755) (width 0.635) (layer F.Cu) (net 10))
 (segment (start 19.685 82.55) (end 19.685 81.915) (width 0.635) (layer F.Cu) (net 10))
 (segment (start 20.32 82.55) (end 19.685 81.915) (width 0.28) (layer F.Cu) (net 10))
 (segment (start 24.13 82.55) (end 20.32 82.55) (width 0.28) (layer F.Cu) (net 10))
 (segment (start 20.32 82.55) (end 19.685 82.55) (width 0.28) (layer F.Cu) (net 10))
 (segment (start 20.32 82.55) (end 19.685 83.185) (width 0.28) (layer F.Cu) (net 10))
 (segment (start 19.685 83.185) (end 19.685 95.885) (width 0.635) (layer F.Cu) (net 10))
 (segment (start 19.685 82.55) (end 19.685 83.185) (width 0.635) (layer F.Cu) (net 10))
 (segment (start 24.191101 49.468899) (end 31.460299 49.468899) (width 0.635) (layer B.Cu) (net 9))
 (segment (start 22.86 50.8) (end 24.191101 49.468899) (width 0.635) (layer B.Cu) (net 9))
 (segment (start 25.4 100.965) (end 21.59 100.965) (width 0.635) (layer B.Cu) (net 9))
 (segment (start 25.4 99.06) (end 25.4 100.965) (width 0.635) (layer B.Cu) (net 9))
 (segment (start 21.59 100.965) (end 19.685 99.06) (width 0.635) (layer B.Cu) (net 9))
 (segment (start 19.685 86.995) (end 22.86 83.82) (width 0.635) (layer B.Cu) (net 9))
 (segment (start 19.685 99.06) (end 19.685 86.995) (width 0.635) (layer B.Cu) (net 9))
 (segment (start 22.86 81.28) (end 19.685 78.105) (width 0.635) (layer B.Cu) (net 9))
 (segment (start 21.3614 50.8) (end 22.86 50.8) (width 0.635) (layer B.Cu) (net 9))
 (segment (start 19.685 52.4764) (end 21.3614 50.8) (width 0.635) (layer B.Cu) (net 9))
 (segment (start 25.4 66.04) (end 24.13 67.31) (width 0.28) (layer B.Cu) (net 9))
 (segment (start 20.32 67.31) (end 19.685 66.675) (width 0.28) (layer B.Cu) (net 9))
 (segment (start 19.685 66.675) (end 19.685 52.4764) (width 0.635) (layer B.Cu) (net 9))
 (segment (start 19.685 67.31) (end 19.685 66.675) (width 0.635) (layer B.Cu) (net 9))
 (segment (start 24.13 67.31) (end 20.32 67.31) (width 0.28) (layer B.Cu) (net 9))
 (segment (start 20.32 67.31) (end 19.685 67.31) (width 0.28) (layer B.Cu) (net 9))
 (segment (start 20.32 67.31) (end 19.685 67.945) (width 0.28) (layer B.Cu) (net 9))
 (segment (start 19.685 67.945) (end 19.685 67.31) (width 0.635) (layer B.Cu) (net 9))
 (segment (start 19.685 78.105) (end 19.685 67.945) (width 0.635) (layer B.Cu) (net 9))
 (segment (start 22.86 83.82) (end 22.86 81.28) (width 0.635) (layer B.Cu) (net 9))
 (segment (start 22.86 81.28) (end 24.13 80.01) (width 0.28) (layer B.Cu) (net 9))
 (segment (start 24.13 80.01) (end 26.035 80.01) (width 0.28) (layer B.Cu) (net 9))
 (segment (start 28.575 80.01) (end 29.845 78.74) (width 0.635) (layer B.Cu) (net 9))
 (segment (start 26.035 80.01) (end 28.575 80.01) (width 0.635) (layer B.Cu) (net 9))
 (segment (start 22.86 73.66) (end 24.13 74.93) (width 0.28) (layer B.Cu) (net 12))
 (segment (start 29.4 77.47) (end 30.48 77.47) (width 0.28) (layer B.Cu) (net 12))
 (segment (start 26.86 74.93) (end 29.4 77.47) (width 0.28) (layer B.Cu) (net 12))
 (segment (start 24.13 74.93) (end 26.86 74.93) (width 0.28) (layer B.Cu) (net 12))
 (segment (start 25.4 93.98) (end 26.667501 95.247501) (width 0.635) (layer B.Cu) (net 21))
 (segment (start 26.263599 93.116401) (end 25.4 93.98) (width 0.28) (layer F.Cu) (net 21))
 (segment (start 26.553601 92.826399) (end 26.263599 93.116401) (width 0.28) (layer F.Cu) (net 21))
 (segment (start 26.553601 73.106271) (end 26.553601 92.826399) (width 0.28) (layer F.Cu) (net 21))
 (via (at 26.035 72.39) (size 0.55) (drill 0.35) (layers F.Cu B.Cu) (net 21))
 (segment (start 26.553601 72.908601) (end 26.035 72.39) (width 0.28) (layer F.Cu) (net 21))
 (segment (start 26.553601 73.106271) (end 26.553601 72.908601) (width 0.28) (layer F.Cu) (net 21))
 (segment (start 24.13 72.39) (end 22.86 71.12) (width 0.28) (layer B.Cu) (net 21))
 (segment (start 26.035 72.39) (end 24.13 72.39) (width 0.28) (layer B.Cu) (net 21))
 (segment (start 22.86 76.2) (end 24.13 74.93) (width 0.28) (layer F.Cu) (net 22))
 (segment (start 24.13 64.77) (end 25.4 63.5) (width 0.28) (layer F.Cu) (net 22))
 (segment (start 24.13 74.93) (end 24.13 64.77) (width 0.28) (layer F.Cu) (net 22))
 (segment (start 25.4 63.5) (end 29.845 63.5) (width 0.28) (layer B.Cu) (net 22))
 (segment (start 29.845 63.5) (end 29.845 63.5) (width 0.28) (layer B.Cu) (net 22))
 (segment (start 23.723599 97.383599) (end 22.86 96.52) (width 0.28) (layer B.Cu) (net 17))
 (segment (start 24.013601 97.673601) (end 23.723599 97.383599) (width 0.28) (layer B.Cu) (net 17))
 (segment (start 29.673399 89.363399) (end 29.916799 89.119999) (width 0.2) (layer B.Cu) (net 19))
 (segment (start 24.13 90.17) (end 27.305 90.17) (width 0.28) (layer B.Cu) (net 19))
 (segment (start 27.305 90.17) (end 28.866798 90.17) (width 0.28) (layer B.Cu) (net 19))
 (segment (start 28.866798 90.17) (end 29.389999 89.646799) (width 0.28) (layer B.Cu) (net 19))
 (segment (start 22.86 91.44) (end 24.13 90.17) (width 0.28) (layer B.Cu) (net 19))
 (segment (start 29.389999 89.646799) (end 29.673399 89.363399) (width 0.28) (layer B.Cu) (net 19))
 (segment (start 27.305 88.9) (end 26.67 88.9) (width 0.28) (layer B.Cu) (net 15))
 (segment (start 27.484999 88.720001) (end 27.305 88.9) (width 0.28) (layer B.Cu) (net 15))
 (segment (start 26.67 88.9) (end 25.4 88.9) (width 0.28) (layer B.Cu) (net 15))
 (segment (start 22.86 88.9) (end 24.13 87.63) (width 0.28) (layer B.Cu) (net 20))
 (segment (start 24.13 87.63) (end 27.305 87.63) (width 0.28) (layer B.Cu) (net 20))
 (segment (start 28.866798 87.63) (end 29.389999 87.106799) (width 0.28) (layer B.Cu) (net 20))
 (segment (start 27.305 87.63) (end 28.866798 87.63) (width 0.28) (layer B.Cu) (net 20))
 (segment (start 29.389999 87.106799) (end 29.673399 86.823399) (width 0.28) (layer B.Cu) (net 20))
 (segment (start 29.673399 86.823399) (end 29.916799 86.579999) (width 0.2) (layer B.Cu) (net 20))
 (segment (start 26.67 86.36) (end 25.4 86.36) (width 0.28) (layer B.Cu) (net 16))
 (segment (start 27.484999 86.180001) (end 27.305 86.36) (width 0.28) (layer B.Cu) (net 16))
 (segment (start 27.305 86.36) (end 26.67 86.36) (width 0.28) (layer B.Cu) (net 16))
 (segment (start 22.86 86.36) (end 24.13 85.09) (width 0.28) (layer B.Cu) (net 18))
 (segment (start 24.13 85.09) (end 27.305 85.09) (width 0.28) (layer B.Cu) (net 18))
 (segment (start 27.305 85.09) (end 28.575 83.82) (width 0.28) (layer B.Cu) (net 18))
 (segment (start 24.13 62.23) (end 35.56 62.23) (width 0.28) (layer B.Cu) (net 5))
 (segment (start 22.86 63.5) (end 24.13 62.23) (width 0.28) (layer B.Cu) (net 5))
 (segment (start 24.13 52.07) (end 35.56 52.07) (width 0.28) (layer B.Cu) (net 8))
 (segment (start 22.86 53.34) (end 24.13 52.07) (width 0.28) (layer B.Cu) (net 8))
 (via (at 27.305 69.85) (size 0.55) (drill 0.35) (layers F.Cu B.Cu) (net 1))
 (segment (start 35.56 69.85) (end 27.305 69.85) (width 0.28) (layer B.Cu) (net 1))
 (segment (start 27.305 60.325) (end 25.4 58.42) (width 0.28) (layer F.Cu) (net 1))
 (segment (start 27.305 69.85) (end 27.305 60.325) (width 0.28) (layer F.Cu) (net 1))
 (segment (start 35.56 67.31) (end 27.94 67.31) (width 0.28) (layer B.Cu) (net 3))
 (via (at 27.94 67.31) (size 0.55) (drill 0.35) (layers F.Cu B.Cu) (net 3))
 (segment (start 27.94 58.42) (end 25.4 55.88) (width 0.28) (layer F.Cu) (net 3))
 (segment (start 27.94 67.31) (end 27.94 58.42) (width 0.28) (layer F.Cu) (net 3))
 (via (at 28.575 64.77) (size 0.55) (drill 0.35) (layers F.Cu B.Cu) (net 4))
 (segment (start 35.56 64.77) (end 28.575 64.77) (width 0.28) (layer B.Cu) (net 4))
 (segment (start 28.575 56.515) (end 25.4 53.34) (width 0.28) (layer F.Cu) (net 4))
 (segment (start 28.575 64.77) (end 28.575 56.515) (width 0.28) (layer F.Cu) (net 4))
 (segment (start 24.13 59.69) (end 35.56 59.69) (width 0.28) (layer B.Cu) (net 2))
 (segment (start 22.86 60.96) (end 24.13 59.69) (width 0.28) (layer B.Cu) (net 2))
 (segment (start 24.13 57.15) (end 35.56 57.15) (width 0.28) (layer B.Cu) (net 6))
 (segment (start 22.86 58.42) (end 24.13 57.15) (width 0.28) (layer B.Cu) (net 6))
 (segment (start 24.13 54.61) (end 22.86 55.88) (width 0.28) (layer B.Cu) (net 7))
 (segment (start 35.56 54.61) (end 24.13 54.61) (width 0.28) (layer B.Cu) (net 7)))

